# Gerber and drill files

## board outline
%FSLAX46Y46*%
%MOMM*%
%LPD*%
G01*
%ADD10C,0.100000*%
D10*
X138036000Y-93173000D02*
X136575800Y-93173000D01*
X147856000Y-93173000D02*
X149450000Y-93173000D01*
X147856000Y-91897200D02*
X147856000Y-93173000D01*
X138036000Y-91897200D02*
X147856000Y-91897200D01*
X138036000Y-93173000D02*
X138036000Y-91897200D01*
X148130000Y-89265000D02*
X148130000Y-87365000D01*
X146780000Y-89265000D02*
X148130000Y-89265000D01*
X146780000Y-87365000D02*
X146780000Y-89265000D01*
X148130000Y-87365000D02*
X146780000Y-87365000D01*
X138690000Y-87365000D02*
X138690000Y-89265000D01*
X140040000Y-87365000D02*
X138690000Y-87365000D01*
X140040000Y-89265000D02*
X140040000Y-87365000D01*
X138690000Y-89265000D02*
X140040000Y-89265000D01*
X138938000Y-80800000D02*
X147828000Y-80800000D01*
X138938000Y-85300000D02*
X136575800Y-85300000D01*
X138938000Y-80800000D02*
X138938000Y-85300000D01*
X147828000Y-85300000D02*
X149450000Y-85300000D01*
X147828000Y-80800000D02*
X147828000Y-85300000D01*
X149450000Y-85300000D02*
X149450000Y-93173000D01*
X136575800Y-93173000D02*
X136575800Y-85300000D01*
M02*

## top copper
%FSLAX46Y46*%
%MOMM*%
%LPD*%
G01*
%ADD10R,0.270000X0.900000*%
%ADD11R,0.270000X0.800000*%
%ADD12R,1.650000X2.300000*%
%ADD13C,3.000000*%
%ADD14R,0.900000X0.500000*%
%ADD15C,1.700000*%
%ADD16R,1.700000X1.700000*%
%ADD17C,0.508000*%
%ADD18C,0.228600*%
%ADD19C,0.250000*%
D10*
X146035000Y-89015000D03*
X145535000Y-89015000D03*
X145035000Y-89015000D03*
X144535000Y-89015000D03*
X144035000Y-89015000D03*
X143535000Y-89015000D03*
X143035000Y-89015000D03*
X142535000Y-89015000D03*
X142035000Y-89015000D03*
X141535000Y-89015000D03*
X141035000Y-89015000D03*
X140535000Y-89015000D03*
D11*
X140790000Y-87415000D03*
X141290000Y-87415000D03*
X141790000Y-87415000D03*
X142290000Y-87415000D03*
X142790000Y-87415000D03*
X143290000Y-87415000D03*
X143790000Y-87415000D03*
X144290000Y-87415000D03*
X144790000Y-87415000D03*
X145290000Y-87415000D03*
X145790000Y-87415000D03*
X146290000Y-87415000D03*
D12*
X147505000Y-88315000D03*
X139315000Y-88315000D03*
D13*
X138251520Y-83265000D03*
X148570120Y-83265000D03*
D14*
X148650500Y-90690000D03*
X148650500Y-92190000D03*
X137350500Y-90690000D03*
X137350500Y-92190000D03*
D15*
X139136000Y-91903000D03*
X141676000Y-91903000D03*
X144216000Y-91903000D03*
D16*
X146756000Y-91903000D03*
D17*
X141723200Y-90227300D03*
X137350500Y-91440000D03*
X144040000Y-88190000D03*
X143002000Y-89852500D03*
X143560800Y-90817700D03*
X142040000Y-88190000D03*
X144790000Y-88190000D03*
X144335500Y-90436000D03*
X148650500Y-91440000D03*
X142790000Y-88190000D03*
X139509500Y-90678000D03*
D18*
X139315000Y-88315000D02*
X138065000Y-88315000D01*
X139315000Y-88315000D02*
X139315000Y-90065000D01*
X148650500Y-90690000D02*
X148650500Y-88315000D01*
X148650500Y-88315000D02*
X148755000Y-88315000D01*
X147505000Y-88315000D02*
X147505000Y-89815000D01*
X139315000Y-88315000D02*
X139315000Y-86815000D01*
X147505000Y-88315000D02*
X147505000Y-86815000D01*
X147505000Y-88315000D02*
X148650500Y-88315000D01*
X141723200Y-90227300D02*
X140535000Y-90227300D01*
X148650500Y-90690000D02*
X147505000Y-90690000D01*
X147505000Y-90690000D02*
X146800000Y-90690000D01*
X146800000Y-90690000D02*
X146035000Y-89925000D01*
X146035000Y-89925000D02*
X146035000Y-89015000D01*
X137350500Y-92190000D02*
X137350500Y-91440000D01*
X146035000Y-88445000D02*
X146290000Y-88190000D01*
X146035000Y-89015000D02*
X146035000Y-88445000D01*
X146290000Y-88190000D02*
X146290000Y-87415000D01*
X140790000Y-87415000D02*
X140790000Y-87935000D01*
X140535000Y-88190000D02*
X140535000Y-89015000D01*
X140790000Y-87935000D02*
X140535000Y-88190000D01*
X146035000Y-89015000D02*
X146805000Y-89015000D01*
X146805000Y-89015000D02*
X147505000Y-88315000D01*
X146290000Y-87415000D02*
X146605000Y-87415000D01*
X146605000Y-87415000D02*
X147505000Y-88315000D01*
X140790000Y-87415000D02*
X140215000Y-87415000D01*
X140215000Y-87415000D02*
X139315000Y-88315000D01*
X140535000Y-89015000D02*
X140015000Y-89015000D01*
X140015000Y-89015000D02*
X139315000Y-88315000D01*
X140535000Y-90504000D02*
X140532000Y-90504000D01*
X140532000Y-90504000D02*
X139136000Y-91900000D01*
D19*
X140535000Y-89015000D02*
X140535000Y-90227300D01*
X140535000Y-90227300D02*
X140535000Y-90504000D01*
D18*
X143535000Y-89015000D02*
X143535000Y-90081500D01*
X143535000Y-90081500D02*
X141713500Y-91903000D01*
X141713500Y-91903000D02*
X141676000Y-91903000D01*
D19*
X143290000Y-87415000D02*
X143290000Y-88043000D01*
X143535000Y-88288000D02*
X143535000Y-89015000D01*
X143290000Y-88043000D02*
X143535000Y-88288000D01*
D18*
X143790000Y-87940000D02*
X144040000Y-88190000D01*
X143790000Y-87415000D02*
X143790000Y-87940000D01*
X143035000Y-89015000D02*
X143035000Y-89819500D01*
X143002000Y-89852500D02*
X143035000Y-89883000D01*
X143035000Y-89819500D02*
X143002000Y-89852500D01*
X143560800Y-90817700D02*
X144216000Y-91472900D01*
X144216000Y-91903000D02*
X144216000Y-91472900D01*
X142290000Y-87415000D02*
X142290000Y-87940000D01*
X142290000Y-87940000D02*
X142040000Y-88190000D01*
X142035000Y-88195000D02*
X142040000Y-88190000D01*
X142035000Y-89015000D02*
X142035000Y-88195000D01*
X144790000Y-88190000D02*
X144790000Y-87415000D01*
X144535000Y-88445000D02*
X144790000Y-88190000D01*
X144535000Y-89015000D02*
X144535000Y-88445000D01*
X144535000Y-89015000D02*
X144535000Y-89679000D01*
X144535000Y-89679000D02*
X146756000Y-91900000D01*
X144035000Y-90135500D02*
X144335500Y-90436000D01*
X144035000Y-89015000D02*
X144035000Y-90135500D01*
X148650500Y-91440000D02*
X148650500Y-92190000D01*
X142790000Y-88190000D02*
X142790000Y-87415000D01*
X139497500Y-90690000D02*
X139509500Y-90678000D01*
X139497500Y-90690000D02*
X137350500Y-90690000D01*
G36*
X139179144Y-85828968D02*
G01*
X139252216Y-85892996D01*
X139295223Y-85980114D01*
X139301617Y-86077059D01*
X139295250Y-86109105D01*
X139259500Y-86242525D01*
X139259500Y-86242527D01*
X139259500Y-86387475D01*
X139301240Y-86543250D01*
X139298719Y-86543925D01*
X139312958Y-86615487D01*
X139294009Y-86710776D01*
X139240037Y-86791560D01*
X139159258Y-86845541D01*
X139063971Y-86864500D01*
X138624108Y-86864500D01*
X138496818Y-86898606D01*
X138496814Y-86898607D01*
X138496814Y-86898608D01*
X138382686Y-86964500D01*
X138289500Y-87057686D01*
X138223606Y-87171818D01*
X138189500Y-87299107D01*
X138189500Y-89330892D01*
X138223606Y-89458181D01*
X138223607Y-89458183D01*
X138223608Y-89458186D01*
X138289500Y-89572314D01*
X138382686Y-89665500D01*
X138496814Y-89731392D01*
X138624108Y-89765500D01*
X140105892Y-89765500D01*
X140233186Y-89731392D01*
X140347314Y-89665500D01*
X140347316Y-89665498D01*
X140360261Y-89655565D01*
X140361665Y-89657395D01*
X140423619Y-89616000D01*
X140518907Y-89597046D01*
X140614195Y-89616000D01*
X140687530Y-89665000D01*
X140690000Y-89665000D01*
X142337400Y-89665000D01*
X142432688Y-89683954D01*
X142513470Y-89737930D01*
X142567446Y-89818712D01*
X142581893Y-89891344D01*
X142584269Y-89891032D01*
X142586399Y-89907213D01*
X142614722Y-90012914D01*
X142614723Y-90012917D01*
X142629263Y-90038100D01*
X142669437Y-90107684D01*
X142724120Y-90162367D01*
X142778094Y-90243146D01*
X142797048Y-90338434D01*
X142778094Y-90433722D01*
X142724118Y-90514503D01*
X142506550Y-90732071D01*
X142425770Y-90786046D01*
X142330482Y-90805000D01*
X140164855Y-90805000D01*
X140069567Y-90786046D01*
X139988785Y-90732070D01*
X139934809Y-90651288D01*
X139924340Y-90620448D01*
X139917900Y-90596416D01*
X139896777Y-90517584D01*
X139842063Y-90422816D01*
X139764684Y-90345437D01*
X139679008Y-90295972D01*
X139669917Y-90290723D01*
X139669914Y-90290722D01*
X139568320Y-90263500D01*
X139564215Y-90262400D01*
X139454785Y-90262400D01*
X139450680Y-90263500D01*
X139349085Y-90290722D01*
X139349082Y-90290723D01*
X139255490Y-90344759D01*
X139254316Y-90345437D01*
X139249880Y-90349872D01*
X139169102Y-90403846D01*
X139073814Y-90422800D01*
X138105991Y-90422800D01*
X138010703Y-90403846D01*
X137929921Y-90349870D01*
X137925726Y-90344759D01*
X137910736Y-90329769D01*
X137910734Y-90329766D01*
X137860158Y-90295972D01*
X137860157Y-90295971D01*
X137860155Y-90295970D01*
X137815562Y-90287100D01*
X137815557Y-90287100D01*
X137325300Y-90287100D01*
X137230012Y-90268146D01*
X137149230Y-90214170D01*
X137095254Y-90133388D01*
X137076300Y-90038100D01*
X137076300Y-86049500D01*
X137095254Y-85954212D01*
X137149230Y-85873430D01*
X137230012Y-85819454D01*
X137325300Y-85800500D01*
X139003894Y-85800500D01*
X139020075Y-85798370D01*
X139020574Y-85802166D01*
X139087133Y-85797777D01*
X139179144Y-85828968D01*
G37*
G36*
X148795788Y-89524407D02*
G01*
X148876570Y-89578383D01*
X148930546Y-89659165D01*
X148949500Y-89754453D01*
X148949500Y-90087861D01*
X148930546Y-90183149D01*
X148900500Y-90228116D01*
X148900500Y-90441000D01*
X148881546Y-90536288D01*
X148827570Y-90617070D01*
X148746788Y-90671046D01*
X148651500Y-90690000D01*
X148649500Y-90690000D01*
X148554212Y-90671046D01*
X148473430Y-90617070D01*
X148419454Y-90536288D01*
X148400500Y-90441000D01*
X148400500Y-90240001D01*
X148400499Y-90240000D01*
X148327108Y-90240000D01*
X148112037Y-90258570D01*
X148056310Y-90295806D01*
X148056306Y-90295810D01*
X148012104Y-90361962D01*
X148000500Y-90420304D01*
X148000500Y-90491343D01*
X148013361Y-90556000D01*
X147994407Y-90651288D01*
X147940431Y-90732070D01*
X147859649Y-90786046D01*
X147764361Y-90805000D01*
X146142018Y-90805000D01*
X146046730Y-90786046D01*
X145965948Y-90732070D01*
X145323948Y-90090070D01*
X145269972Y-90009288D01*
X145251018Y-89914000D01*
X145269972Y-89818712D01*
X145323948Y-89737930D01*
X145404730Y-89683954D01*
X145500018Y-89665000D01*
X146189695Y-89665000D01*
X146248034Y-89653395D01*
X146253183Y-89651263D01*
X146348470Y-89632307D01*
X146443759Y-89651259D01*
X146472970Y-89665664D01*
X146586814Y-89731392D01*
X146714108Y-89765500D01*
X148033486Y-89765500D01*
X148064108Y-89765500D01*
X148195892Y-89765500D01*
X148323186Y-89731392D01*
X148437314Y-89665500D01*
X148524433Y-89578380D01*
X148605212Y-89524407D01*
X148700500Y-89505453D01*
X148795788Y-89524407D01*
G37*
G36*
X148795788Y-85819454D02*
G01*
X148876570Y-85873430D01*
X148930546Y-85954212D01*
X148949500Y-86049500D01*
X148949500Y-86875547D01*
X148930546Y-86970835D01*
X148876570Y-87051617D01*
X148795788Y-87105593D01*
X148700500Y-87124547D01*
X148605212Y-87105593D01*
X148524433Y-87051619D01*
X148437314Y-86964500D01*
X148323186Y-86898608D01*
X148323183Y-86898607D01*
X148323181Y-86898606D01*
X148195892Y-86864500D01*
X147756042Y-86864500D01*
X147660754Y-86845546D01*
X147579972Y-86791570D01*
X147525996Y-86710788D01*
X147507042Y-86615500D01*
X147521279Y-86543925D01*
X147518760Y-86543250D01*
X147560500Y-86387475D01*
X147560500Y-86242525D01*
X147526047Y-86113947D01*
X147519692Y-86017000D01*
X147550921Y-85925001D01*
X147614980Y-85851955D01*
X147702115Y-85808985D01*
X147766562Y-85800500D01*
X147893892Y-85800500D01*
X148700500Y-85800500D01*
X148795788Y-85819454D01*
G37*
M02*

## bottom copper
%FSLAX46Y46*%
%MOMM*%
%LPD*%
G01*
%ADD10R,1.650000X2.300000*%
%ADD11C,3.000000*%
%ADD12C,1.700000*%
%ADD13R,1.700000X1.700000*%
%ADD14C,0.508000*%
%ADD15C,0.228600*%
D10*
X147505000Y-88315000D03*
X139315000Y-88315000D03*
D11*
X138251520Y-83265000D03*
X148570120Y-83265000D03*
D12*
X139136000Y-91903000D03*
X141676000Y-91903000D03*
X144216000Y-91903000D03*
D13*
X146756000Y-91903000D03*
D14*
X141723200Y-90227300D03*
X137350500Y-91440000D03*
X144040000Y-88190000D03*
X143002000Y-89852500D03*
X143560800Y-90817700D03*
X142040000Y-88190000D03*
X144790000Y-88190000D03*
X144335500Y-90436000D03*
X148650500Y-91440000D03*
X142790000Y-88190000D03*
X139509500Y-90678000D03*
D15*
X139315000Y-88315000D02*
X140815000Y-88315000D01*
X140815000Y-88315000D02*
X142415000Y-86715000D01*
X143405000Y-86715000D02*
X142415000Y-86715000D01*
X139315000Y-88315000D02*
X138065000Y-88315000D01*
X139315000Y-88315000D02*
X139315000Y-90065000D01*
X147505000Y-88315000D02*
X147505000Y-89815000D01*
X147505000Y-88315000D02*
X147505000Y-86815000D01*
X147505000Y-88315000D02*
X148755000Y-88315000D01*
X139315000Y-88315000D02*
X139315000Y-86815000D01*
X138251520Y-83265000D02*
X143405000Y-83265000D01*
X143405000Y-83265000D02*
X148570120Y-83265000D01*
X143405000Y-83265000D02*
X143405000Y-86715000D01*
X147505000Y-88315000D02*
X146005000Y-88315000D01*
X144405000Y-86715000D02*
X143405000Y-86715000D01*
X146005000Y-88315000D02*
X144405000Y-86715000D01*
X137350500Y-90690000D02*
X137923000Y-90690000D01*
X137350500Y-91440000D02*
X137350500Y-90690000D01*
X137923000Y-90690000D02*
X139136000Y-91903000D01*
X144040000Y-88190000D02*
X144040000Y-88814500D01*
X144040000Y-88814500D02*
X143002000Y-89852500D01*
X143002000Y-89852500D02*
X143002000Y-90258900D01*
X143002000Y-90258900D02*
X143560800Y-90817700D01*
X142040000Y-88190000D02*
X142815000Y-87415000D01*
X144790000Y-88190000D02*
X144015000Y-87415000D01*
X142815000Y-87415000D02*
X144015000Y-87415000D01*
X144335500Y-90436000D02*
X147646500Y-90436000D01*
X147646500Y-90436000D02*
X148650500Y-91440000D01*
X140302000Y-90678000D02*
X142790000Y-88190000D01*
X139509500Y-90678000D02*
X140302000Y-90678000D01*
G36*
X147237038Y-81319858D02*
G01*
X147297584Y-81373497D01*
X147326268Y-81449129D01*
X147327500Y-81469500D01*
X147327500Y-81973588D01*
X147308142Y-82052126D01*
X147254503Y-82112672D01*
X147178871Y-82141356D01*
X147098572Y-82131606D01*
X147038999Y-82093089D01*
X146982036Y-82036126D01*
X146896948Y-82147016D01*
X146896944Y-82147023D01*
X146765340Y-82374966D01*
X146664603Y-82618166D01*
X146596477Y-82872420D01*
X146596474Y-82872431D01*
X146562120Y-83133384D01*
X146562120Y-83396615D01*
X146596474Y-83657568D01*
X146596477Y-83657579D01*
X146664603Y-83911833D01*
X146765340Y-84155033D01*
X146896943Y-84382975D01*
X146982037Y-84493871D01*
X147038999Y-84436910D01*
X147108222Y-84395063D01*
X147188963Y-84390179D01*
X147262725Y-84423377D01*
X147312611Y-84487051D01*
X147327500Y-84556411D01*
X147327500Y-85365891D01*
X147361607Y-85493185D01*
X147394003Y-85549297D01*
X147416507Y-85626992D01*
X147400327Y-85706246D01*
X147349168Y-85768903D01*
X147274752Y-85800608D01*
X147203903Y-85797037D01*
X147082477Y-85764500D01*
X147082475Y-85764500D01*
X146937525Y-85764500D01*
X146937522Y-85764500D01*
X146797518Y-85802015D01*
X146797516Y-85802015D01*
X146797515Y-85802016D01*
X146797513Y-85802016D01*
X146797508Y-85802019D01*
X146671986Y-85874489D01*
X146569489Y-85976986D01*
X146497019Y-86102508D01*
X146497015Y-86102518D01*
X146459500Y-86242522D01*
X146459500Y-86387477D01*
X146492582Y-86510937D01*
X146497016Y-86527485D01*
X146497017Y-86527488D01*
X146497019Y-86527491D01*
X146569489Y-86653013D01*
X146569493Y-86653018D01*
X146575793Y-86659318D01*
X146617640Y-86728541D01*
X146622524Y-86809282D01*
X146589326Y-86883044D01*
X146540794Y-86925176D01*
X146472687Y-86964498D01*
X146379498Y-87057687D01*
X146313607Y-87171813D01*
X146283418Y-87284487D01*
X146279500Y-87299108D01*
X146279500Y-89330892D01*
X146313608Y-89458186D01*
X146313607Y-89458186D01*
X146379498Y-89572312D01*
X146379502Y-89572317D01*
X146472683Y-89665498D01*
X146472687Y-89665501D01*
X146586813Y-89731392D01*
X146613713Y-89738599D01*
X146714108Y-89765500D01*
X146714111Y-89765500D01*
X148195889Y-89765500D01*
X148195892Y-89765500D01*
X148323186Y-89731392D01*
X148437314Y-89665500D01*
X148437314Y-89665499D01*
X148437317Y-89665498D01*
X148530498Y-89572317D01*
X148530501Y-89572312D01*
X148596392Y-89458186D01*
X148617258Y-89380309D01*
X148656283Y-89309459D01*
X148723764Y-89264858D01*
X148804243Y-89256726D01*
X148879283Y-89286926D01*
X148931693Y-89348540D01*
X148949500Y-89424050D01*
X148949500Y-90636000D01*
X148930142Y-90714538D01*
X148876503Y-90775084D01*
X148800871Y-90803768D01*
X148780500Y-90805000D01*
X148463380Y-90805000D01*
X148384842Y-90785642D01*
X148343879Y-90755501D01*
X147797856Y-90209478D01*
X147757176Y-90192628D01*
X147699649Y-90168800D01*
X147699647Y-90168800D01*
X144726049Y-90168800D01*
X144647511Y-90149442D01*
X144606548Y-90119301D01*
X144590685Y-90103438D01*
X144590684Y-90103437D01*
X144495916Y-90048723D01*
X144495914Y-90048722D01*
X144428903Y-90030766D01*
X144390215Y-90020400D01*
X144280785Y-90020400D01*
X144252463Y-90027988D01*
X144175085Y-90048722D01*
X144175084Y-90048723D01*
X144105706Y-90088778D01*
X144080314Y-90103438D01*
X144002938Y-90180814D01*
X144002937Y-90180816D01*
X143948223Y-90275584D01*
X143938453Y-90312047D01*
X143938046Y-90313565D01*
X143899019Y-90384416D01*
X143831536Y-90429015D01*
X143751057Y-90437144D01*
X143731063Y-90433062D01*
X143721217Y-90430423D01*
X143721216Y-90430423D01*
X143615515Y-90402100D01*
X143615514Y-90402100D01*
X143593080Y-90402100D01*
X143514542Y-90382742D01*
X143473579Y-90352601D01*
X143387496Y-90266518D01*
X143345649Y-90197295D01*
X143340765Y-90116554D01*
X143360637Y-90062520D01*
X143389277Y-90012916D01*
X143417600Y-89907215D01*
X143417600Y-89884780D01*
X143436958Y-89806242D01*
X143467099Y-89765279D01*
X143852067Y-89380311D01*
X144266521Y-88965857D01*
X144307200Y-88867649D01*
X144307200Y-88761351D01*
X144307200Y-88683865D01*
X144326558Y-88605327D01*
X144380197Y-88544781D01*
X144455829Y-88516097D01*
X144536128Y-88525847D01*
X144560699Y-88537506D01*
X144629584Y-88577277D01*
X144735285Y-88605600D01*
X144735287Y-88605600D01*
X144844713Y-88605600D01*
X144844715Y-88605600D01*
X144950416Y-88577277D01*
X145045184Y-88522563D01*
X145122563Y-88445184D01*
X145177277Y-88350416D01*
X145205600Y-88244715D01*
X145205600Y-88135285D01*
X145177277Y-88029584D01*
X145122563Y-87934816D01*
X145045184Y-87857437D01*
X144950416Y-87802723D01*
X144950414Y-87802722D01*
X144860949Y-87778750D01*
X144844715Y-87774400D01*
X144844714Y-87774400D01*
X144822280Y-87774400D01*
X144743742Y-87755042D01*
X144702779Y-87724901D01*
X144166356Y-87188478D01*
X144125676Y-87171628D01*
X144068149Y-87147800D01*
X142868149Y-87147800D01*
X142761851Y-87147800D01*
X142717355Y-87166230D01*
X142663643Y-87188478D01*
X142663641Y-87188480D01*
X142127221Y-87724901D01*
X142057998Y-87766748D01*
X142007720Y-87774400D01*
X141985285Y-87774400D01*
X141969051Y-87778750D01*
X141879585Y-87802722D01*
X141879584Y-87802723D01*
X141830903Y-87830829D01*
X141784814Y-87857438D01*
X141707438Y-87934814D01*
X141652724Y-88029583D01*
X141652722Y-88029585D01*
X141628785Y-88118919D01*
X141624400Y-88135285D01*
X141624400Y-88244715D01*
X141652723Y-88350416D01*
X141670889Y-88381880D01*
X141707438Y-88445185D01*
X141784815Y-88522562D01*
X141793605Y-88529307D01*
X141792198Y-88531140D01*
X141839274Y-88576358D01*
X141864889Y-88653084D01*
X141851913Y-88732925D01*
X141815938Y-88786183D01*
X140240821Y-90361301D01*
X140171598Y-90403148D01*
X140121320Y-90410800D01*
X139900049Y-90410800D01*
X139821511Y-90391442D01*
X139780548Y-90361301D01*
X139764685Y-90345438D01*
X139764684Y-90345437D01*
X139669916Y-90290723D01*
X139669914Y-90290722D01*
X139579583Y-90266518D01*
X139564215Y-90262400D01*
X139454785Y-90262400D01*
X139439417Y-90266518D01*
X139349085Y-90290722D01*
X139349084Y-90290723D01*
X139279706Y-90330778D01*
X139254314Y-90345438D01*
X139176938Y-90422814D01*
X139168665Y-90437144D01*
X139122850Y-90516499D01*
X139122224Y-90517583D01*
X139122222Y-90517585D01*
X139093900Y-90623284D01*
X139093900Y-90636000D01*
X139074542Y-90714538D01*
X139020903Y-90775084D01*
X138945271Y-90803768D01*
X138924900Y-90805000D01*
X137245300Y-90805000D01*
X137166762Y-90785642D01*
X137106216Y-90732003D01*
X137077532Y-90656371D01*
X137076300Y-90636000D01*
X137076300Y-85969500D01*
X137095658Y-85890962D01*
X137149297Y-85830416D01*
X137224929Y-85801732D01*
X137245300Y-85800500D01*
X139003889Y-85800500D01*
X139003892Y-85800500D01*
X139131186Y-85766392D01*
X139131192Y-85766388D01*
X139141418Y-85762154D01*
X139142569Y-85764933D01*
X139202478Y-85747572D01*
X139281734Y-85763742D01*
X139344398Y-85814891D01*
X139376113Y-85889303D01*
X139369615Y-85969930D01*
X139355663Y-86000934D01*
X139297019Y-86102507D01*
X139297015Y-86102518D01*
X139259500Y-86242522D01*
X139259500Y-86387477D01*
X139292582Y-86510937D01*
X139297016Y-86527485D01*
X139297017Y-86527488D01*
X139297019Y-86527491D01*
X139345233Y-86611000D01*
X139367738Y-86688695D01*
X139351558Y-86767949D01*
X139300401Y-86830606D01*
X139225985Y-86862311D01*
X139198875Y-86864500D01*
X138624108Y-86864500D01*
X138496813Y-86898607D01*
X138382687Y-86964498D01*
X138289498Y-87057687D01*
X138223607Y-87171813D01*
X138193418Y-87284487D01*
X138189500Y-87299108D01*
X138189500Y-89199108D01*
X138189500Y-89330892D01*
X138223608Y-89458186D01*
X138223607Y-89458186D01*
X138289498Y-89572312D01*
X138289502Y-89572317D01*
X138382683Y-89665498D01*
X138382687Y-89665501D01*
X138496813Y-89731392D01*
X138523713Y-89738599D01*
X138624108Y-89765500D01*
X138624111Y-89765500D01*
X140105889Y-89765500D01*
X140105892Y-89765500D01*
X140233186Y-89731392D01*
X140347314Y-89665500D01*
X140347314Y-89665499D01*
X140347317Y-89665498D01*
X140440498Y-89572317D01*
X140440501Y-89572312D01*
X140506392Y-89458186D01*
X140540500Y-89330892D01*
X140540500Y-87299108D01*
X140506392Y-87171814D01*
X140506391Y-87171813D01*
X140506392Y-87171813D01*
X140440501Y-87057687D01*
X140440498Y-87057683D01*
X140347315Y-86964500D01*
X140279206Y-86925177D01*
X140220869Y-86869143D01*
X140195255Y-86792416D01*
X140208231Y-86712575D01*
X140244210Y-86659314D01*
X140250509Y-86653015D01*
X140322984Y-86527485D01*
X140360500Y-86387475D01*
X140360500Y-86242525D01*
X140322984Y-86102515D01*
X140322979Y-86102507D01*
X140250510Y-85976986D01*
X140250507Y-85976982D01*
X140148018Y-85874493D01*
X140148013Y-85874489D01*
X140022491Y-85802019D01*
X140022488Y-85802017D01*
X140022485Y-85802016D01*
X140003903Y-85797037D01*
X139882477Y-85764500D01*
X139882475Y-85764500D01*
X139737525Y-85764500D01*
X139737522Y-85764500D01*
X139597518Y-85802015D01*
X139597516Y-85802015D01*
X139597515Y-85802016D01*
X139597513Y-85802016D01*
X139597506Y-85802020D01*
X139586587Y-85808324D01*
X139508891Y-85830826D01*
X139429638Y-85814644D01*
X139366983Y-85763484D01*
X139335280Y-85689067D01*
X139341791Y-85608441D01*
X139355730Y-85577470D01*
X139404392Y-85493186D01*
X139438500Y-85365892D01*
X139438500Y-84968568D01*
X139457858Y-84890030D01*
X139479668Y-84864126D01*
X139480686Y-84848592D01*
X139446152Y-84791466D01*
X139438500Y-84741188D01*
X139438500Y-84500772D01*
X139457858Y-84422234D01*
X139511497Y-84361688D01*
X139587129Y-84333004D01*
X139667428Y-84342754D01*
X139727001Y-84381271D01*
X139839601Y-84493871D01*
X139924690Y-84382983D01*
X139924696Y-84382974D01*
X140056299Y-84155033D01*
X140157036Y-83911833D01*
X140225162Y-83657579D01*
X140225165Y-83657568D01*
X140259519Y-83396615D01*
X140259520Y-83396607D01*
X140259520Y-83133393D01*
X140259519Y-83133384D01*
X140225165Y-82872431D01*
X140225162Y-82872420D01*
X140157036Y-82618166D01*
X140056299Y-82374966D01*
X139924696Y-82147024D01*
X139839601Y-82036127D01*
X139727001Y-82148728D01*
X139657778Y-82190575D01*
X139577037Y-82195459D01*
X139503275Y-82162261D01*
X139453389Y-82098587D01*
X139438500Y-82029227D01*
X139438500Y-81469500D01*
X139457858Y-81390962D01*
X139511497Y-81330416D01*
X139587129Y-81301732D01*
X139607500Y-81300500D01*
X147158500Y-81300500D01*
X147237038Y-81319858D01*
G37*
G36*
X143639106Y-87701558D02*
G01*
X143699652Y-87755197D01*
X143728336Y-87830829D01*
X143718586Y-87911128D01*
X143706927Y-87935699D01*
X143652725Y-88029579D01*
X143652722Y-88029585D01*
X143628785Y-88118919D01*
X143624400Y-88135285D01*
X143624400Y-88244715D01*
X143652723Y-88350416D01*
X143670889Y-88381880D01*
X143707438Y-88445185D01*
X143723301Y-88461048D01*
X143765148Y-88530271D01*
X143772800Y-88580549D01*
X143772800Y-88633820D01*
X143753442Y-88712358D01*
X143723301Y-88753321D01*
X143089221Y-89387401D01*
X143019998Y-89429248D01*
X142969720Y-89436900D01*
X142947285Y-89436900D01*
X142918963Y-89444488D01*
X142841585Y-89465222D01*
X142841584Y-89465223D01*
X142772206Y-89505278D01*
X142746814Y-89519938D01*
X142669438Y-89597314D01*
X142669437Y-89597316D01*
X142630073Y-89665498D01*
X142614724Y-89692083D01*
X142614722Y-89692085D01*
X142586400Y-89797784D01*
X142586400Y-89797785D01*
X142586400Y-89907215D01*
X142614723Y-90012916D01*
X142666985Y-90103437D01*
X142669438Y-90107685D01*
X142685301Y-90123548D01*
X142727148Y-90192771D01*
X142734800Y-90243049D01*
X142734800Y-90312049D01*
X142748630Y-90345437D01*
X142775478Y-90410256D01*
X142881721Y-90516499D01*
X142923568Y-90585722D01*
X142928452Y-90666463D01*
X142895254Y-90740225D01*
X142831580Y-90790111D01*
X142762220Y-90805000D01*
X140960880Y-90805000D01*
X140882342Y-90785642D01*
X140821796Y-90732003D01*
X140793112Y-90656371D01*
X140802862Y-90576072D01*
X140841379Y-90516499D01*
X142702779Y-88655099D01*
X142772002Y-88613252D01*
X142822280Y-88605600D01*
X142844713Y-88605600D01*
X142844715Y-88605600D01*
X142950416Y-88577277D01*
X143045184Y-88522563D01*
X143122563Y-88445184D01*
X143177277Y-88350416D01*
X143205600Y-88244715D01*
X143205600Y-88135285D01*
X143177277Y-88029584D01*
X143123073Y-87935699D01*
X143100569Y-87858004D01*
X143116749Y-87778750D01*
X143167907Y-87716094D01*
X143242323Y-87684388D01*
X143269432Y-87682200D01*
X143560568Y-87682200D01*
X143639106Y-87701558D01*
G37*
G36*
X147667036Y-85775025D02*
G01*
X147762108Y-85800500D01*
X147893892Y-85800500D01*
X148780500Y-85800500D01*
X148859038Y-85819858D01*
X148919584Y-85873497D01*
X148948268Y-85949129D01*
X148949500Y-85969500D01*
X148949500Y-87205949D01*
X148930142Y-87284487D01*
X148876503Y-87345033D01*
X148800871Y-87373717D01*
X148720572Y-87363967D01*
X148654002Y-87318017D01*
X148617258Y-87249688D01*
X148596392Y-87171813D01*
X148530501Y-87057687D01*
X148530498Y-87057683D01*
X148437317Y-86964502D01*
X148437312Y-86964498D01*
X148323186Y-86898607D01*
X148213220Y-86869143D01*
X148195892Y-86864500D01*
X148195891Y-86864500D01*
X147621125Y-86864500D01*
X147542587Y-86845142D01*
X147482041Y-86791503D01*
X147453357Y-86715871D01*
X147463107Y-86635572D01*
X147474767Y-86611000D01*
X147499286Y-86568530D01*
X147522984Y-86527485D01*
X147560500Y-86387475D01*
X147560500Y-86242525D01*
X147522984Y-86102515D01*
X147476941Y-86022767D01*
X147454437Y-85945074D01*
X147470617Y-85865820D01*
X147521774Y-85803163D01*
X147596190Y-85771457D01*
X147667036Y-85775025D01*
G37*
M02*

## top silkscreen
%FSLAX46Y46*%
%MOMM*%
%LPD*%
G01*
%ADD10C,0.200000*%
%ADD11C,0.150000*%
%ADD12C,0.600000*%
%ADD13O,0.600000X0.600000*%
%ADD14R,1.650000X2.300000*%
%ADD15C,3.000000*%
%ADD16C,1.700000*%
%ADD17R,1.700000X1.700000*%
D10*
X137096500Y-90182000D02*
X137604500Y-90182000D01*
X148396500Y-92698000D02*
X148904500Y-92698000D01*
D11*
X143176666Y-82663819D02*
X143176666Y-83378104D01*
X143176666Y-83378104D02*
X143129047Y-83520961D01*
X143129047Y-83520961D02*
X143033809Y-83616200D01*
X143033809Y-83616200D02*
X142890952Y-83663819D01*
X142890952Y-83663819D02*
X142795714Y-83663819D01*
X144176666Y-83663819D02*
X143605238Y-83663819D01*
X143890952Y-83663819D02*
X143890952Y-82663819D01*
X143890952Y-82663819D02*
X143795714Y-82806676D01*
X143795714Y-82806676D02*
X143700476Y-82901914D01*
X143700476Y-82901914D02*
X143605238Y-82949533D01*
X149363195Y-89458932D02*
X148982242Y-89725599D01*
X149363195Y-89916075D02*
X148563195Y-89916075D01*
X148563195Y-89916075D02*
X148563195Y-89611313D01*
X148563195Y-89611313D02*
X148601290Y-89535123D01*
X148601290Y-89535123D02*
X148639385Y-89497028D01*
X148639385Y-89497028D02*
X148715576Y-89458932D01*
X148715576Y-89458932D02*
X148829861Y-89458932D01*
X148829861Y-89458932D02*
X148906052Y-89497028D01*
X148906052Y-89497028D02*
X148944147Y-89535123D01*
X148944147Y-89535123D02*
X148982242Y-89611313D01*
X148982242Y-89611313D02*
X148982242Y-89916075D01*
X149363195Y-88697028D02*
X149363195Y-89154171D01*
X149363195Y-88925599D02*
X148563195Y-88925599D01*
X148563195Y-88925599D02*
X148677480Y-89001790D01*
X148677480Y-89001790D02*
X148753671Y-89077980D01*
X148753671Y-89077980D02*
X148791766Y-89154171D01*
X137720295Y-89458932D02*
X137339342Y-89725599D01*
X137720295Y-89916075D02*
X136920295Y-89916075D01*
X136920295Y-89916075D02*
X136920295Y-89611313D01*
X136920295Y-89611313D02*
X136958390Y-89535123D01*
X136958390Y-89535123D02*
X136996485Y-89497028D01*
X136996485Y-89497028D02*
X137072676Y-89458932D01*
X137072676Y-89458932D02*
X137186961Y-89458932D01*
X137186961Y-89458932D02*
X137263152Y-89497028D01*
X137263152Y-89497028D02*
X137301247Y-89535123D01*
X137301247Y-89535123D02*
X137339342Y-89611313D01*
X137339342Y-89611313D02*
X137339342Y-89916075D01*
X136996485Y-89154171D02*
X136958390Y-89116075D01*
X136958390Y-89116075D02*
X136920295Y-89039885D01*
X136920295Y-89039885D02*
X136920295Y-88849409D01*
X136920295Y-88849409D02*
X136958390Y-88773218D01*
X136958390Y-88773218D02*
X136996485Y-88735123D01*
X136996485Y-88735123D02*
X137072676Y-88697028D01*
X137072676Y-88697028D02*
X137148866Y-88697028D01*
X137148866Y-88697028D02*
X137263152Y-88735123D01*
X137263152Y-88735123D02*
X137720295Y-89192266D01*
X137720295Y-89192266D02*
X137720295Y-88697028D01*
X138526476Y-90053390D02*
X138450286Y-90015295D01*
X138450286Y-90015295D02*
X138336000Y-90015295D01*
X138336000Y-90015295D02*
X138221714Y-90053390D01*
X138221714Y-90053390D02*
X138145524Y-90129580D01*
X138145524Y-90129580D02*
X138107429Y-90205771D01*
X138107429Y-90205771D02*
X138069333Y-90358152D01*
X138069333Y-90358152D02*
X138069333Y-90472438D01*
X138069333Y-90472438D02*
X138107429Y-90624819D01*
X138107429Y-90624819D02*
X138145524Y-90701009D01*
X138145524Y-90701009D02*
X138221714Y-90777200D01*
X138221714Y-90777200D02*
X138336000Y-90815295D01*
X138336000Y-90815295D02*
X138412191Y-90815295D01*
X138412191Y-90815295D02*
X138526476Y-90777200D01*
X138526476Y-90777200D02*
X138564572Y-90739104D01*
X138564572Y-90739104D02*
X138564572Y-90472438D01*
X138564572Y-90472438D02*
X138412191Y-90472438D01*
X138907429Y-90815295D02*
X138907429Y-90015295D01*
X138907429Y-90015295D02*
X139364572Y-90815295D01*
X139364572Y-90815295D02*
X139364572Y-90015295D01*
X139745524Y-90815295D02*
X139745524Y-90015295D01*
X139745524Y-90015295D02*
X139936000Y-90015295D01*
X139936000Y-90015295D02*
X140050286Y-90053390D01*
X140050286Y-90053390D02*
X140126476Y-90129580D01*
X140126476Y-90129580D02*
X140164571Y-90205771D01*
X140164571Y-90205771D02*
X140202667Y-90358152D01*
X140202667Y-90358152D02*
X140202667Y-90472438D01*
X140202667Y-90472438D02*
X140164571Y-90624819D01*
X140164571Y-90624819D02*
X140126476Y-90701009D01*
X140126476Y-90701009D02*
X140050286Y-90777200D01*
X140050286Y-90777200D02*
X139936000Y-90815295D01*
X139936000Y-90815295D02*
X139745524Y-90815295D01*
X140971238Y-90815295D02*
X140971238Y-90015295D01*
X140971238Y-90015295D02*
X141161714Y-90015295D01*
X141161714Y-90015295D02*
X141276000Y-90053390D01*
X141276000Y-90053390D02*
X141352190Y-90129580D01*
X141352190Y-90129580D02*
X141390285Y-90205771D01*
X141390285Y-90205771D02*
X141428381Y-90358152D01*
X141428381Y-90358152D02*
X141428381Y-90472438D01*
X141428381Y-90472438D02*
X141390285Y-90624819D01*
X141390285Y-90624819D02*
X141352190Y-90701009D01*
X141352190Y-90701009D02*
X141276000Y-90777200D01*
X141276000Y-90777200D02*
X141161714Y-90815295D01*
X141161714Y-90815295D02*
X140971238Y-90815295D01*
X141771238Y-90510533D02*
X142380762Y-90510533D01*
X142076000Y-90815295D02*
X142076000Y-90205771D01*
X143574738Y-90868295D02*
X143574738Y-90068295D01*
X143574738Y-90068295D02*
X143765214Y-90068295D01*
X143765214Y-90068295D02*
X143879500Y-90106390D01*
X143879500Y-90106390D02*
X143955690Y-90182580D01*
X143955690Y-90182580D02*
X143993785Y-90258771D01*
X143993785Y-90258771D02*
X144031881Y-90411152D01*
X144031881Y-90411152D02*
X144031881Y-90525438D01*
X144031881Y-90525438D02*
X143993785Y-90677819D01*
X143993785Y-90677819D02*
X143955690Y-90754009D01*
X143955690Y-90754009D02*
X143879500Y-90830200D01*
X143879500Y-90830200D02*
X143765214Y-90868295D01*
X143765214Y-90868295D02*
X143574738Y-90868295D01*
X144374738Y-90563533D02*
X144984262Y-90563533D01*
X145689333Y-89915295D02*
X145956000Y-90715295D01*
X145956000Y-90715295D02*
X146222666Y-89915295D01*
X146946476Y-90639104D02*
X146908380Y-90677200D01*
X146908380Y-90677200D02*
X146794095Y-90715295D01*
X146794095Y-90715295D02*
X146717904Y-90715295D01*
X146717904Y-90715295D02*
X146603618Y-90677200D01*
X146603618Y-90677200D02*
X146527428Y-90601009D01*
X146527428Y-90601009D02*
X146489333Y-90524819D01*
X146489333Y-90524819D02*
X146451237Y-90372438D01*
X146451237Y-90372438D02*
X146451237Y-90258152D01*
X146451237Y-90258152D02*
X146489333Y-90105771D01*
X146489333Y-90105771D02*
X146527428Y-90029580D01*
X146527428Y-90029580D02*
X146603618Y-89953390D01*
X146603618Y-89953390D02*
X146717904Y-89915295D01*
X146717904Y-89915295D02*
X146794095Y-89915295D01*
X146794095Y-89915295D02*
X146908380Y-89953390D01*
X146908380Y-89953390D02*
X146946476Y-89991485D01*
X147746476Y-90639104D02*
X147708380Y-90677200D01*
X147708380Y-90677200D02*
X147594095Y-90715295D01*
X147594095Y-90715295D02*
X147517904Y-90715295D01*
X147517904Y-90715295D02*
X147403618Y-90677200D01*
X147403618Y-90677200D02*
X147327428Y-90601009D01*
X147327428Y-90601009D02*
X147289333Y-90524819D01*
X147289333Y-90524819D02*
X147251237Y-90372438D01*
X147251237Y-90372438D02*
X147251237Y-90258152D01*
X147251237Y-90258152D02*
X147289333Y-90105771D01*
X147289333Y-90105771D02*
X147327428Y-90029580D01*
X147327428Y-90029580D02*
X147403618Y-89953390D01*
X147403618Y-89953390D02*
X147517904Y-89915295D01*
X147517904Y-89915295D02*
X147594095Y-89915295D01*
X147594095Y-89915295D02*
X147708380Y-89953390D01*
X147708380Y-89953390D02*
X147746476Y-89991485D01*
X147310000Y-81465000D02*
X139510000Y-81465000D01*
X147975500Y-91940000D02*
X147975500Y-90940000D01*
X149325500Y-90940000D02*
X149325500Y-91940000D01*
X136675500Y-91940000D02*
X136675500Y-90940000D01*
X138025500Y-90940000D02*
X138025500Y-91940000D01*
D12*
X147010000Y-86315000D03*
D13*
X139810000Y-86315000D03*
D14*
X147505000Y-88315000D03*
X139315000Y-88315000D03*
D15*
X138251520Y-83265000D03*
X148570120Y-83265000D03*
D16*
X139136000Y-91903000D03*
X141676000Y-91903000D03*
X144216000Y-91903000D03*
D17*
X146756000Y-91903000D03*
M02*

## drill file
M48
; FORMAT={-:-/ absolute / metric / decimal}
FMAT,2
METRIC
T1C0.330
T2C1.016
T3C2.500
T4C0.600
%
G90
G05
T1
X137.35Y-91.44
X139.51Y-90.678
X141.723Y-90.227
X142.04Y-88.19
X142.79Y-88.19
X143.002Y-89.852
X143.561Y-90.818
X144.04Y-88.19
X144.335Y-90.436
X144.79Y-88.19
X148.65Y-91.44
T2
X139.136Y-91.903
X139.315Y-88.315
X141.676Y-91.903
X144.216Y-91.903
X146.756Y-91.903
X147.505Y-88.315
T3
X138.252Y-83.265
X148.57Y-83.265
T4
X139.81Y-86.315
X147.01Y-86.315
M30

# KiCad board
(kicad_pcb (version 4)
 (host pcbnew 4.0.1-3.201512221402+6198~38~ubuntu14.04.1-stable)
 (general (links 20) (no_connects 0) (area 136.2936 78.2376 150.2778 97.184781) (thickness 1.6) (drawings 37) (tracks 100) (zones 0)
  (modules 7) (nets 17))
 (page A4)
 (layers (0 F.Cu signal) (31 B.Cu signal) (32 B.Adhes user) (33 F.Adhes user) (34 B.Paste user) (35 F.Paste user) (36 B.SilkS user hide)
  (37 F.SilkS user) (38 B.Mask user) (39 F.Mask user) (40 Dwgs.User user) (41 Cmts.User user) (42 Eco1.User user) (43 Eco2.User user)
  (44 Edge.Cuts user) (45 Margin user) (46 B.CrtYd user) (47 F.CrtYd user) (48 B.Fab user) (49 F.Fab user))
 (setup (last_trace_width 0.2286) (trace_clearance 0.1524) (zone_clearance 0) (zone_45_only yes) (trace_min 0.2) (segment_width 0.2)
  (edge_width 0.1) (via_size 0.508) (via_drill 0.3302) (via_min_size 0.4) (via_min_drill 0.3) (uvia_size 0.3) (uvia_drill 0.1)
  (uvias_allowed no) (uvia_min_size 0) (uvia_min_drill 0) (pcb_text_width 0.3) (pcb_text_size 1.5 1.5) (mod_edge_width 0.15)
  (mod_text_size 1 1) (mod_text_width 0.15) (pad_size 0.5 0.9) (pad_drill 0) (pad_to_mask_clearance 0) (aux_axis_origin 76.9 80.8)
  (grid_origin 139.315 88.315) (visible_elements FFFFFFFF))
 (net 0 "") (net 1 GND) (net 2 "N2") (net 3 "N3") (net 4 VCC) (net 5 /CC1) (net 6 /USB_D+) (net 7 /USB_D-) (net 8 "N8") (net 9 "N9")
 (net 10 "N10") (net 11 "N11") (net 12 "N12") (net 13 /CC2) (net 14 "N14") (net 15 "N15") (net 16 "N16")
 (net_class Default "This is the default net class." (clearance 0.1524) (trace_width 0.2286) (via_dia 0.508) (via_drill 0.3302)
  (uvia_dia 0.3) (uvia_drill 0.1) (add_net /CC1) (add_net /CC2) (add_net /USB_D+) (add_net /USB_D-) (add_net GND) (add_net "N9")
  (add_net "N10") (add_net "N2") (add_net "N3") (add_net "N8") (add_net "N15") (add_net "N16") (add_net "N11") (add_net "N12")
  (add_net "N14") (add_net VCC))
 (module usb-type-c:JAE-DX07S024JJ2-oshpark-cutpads (layer F.Cu) (at 147.01 86.315 180)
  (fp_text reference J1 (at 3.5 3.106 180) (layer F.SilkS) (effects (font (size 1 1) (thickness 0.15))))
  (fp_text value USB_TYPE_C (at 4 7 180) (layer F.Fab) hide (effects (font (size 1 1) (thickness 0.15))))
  (fp_line (start -0.3 4.85) (end 7.5 4.85) (layer F.SilkS) (width 0.15))
  (pad A1 smd rect (at 0.975 -2.7 180) (size 0.27 0.9) (layers F.Cu F.Paste F.Mask) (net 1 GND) (zone_connect 1) (thermal_width 0.2)
   (thermal_gap 0.2))
  (pad A2 smd rect (at 1.475 -2.7 180) (size 0.27 0.9) (layers F.Cu F.Paste F.Mask) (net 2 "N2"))
  (pad A3 smd rect (at 1.975 -2.7 180) (size 0.27 0.9) (layers F.Cu F.Paste F.Mask) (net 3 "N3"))
  (pad A4 smd rect (at 2.475 -2.7 180) (size 0.27 0.9) (layers F.Cu F.Paste F.Mask) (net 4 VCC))
  (pad A5 smd rect (at 2.975 -2.7 180) (size 0.27 0.9) (layers F.Cu F.Paste F.Mask) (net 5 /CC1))
  (pad A6 smd rect (at 3.475 -2.7 180) (size 0.27 0.9) (layers F.Cu F.Paste F.Mask) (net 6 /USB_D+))
  (pad A7 smd rect (at 3.975 -2.7 180) (size 0.27 0.9) (layers F.Cu F.Paste F.Mask) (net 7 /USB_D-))
  (pad A8 smd rect (at 4.475 -2.7 180) (size 0.27 0.9) (layers F.Cu F.Paste F.Mask) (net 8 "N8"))
  (pad A9 smd rect (at 4.975 -2.7 180) (size 0.27 0.9) (layers F.Cu F.Paste F.Mask) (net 4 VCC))
  (pad A10 smd rect (at 5.475 -2.7 180) (size 0.27 0.9) (layers F.Cu F.Paste F.Mask) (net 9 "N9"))
  (pad A11 smd rect (at 5.975 -2.7 180) (size 0.27 0.9) (layers F.Cu F.Paste F.Mask) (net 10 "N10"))
  (pad A12 smd rect (at 6.475 -2.7 180) (size 0.27 0.9) (layers F.Cu F.Paste F.Mask) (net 1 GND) (zone_connect 2))
  (pad B1 smd rect (at 6.22 -1.1 180) (size 0.27 0.8) (layers F.Cu F.Paste F.Mask) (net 1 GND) (zone_connect 2))
  (pad B2 smd rect (at 5.72 -1.1 180) (size 0.27 0.8) (layers F.Cu F.Paste F.Mask) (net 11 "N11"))
  (pad B3 smd rect (at 5.22 -1.1 180) (size 0.27 0.8) (layers F.Cu F.Paste F.Mask) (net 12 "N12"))
  (pad B4 smd rect (at 4.72 -1.1 180) (size 0.27 0.8) (layers F.Cu F.Paste F.Mask) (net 4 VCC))
  (pad B5 smd rect (at 4.22 -1.1 180) (size 0.27 0.8) (layers F.Cu F.Paste F.Mask) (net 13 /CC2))
  (pad B6 smd rect (at 3.72 -1.1 180) (size 0.27 0.8) (layers F.Cu F.Paste F.Mask) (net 6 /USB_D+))
  (pad B7 smd rect (at 3.22 -1.1 180) (size 0.27 0.8) (layers F.Cu F.Paste F.Mask) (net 7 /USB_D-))
  (pad B8 smd rect (at 2.72 -1.1 180) (size 0.27 0.8) (layers F.Cu F.Paste F.Mask) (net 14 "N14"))
  (pad B9 smd rect (at 2.22 -1.1 180) (size 0.27 0.8) (layers F.Cu F.Paste F.Mask) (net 4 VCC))
  (pad B10 smd rect (at 1.72 -1.1 180) (size 0.27 0.8) (layers F.Cu F.Paste F.Mask) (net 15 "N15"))
  (pad B11 smd rect (at 1.22 -1.1 180) (size 0.27 0.8) (layers F.Cu F.Paste F.Mask) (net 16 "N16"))
  (pad B12 smd rect (at 0.72 -1.1 180) (size 0.27 0.8) (layers F.Cu F.Paste F.Mask) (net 1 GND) (zone_connect 2))
  (pad "" np_thru_hole circle (at 0 0 180) (size 0.6 0.6) (drill 0.6) (layers *.Cu *.Mask F.SilkS))
  (pad "" np_thru_hole oval (at 7.2 0 180) (size 0.6 0.6) (drill 0.6) (layers *.Cu *.Mask F.SilkS))
  (pad 0 thru_hole rect (at -0.495 -2 180) (size 1.65 2.3) (drill 1.016) (layers *.Cu *.Mask F.SilkS) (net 1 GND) (zone_connect 1)
   (thermal_width 0.2) (thermal_gap 0.2))
  (pad 0 thru_hole rect (at 7.695 -2 180) (size 1.65 2.3) (drill 1.016) (layers *.Cu *.Mask F.SilkS) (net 1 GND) (zone_connect 1)
   (thermal_width 0.2) (thermal_gap 0.2))
  (pad 0 thru_hole circle (at 8.75848 3.05 180) (size 3 3) (drill 2.5) (layers *.Cu *.Mask F.SilkS) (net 1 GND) (zone_connect 1))
  (pad 0 thru_hole circle (at -1.56012 3.05 180) (size 3 3) (drill 2.5) (layers *.Cu *.Mask F.SilkS) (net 1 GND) (zone_connect 1)))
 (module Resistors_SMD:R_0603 (layer F.Cu) (at 148.6505 91.44 270)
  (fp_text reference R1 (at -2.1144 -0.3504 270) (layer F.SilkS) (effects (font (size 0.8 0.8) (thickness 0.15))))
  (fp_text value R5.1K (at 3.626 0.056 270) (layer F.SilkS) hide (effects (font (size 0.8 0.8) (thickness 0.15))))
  (fp_line (start 0.5 0.675) (end -0.5 0.675) (layer F.SilkS) (width 0.15))
  (fp_line (start -0.5 -0.675) (end 0.5 -0.675) (layer F.SilkS) (width 0.15))
  (pad 1 smd rect (at -0.75 0 270) (size 0.5 0.9) (layers F.Cu F.Paste F.Mask) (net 1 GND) (zone_connect 1) (thermal_width 0.2)
   (thermal_gap 0.2))
  (pad 2 smd rect (at 0.75 0 270) (size 0.5 0.9) (layers F.Cu F.Paste F.Mask) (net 5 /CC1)))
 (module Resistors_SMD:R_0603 (layer F.Cu) (at 137.3505 91.44 270)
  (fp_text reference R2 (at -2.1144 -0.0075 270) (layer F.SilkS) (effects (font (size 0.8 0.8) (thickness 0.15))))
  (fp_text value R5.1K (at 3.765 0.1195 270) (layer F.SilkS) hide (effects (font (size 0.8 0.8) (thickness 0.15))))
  (fp_line (start 0.5 0.675) (end -0.5 0.675) (layer F.SilkS) (width 0.15))
  (fp_line (start -0.5 -0.675) (end 0.5 -0.675) (layer F.SilkS) (width 0.15))
  (pad 1 smd rect (at -0.75 0 270) (size 0.5 0.9) (layers F.Cu F.Paste F.Mask) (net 13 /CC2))
  (pad 2 smd rect (at 0.75 0 270) (size 0.5 0.9) (layers F.Cu F.Paste F.Mask) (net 1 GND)))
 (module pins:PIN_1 (layer F.Cu) (at 139.136 91.903)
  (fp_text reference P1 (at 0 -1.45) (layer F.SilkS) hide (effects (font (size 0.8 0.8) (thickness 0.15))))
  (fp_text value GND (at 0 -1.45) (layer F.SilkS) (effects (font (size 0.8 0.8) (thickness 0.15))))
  (pad 1 thru_hole circle (at 0 0) (size 1.7 1.7) (drill 1.016) (layers *.Cu *.Mask F.SilkS) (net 1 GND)))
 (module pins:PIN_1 (layer F.Cu) (at 141.676 91.903)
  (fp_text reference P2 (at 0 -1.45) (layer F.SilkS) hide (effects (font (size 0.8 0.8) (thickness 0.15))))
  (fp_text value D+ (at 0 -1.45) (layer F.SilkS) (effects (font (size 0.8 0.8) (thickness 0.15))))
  (pad 1 thru_hole circle (at 0 0) (size 1.7 1.7) (drill 1.016) (layers *.Cu *.Mask F.SilkS) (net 6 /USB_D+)))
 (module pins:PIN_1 (layer F.Cu) (at 144.216 91.903 90)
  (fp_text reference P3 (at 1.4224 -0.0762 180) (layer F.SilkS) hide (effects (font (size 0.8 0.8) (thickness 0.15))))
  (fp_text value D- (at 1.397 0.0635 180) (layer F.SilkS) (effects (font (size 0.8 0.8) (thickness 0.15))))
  (pad 1 thru_hole circle (at 0 0 90) (size 1.7 1.7) (drill 1.016) (layers *.Cu *.Mask F.SilkS) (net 7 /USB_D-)))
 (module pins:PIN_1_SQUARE (layer F.Cu) (at 146.756 91.903)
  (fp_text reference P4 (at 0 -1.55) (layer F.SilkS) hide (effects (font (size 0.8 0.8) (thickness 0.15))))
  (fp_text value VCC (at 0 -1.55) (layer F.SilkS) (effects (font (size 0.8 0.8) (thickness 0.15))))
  (pad 1 thru_hole rect (at 0 0) (size 1.7 1.7) (drill 1.016) (layers *.Cu *.Mask F.SilkS) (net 4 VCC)))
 (gr_line (start 137.0965 90.182) (end 137.6045 90.182) (angle 90) (layer F.SilkS) (width 0.2))
 (gr_line (start 148.3965 92.698) (end 148.9045 92.698) (angle 90) (layer F.SilkS) (width 0.2))
 (gr_line (start 138.036 93.173) (end 136.5758 93.173) (angle 90) (layer Edge.Cuts) (width 0.1))
 (gr_line (start 147.856 93.173) (end 149.45 93.173) (angle 90) (layer Edge.Cuts) (width 0.1))
 (gr_line (start 147.856 91.8972) (end 147.856 93.173) (angle 90) (layer Edge.Cuts) (width 0.1))
 (gr_line (start 138.036 91.8972) (end 147.856 91.8972) (angle 90) (layer Edge.Cuts) (width 0.1))
 (gr_line (start 138.036 93.173) (end 138.036 91.8972) (angle 90) (layer Edge.Cuts) (width 0.1))
 (gr_line (start 148.13 89.265) (end 148.13 87.365) (angle 90) (layer Edge.Cuts) (width 0.1))
 (gr_line (start 146.78 89.265) (end 148.13 89.265) (angle 90) (layer Edge.Cuts) (width 0.1))
 (gr_line (start 146.78 87.365) (end 146.78 89.265) (angle 90) (layer Edge.Cuts) (width 0.1))
 (gr_line (start 148.13 87.365) (end 146.78 87.365) (angle 90) (layer Edge.Cuts) (width 0.1))
 (gr_line (start 138.69 87.365) (end 138.69 89.265) (angle 90) (layer Edge.Cuts) (width 0.1))
 (gr_line (start 140.04 87.365) (end 138.69 87.365) (angle 90) (layer Edge.Cuts) (width 0.1))
 (gr_line (start 140.04 89.265) (end 140.04 87.365) (angle 90) (layer Edge.Cuts) (width 0.1))
 (gr_line (start 138.69 89.265) (end 140.04 89.265) (angle 90) (layer Edge.Cuts) (width 0.1))
 (gr_line (start 138.938 80.8) (end 147.828 80.8) (angle 90) (layer Edge.Cuts) (width 0.1))
 (gr_line (start 138.938 85.3) (end 136.5758 85.3) (angle 90) (layer Edge.Cuts) (width 0.1))
 (gr_line (start 138.938 80.8) (end 138.938 85.3) (angle 90) (layer Edge.Cuts) (width 0.1))
 (gr_line (start 147.828 85.3) (end 149.45 85.3) (angle 90) (layer Edge.Cuts) (width 0.1))
 (gr_line (start 147.828 80.8) (end 147.828 85.3) (angle 90) (layer Edge.Cuts) (width 0.1))
 (gr_line (start 149.45 85.3) (end 149.45 93.173) (angle 90) (layer Edge.Cuts) (width 0.1))
 (gr_line (start 136.5758 93.173) (end 136.5758 85.3) (angle 90) (layer Edge.Cuts) (width 0.1))
 (segment (start 139.315 88.315) (end 140.815 88.315) (width 0.2286) (layer B.Cu) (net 1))
 (segment (start 140.815 88.315) (end 142.415 86.715) (width 0.2286) (layer B.Cu) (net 1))
 (segment (start 143.405 86.715) (end 142.415 86.715) (width 0.2286) (layer B.Cu) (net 1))
 (segment (start 139.315 88.315) (end 138.065 88.315) (width 0.2286) (layer B.Cu) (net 1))
 (segment (start 139.315 88.315) (end 138.065 88.315) (width 0.2286) (layer F.Cu) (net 1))
 (segment (start 139.315 88.315) (end 139.315 90.065) (width 0.2286) (layer B.Cu) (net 1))
 (segment (start 147.505 88.315) (end 147.505 89.815) (width 0.2286) (layer B.Cu) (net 1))
 (segment (start 147.505 88.315) (end 147.505 86.815) (width 0.2286) (layer B.Cu) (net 1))
 (segment (start 147.505 88.315) (end 148.755 88.315) (width 0.2286) (layer B.Cu) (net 1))
 (segment (start 139.315 88.315) (end 139.315 86.815) (width 0.2286) (layer B.Cu) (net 1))
 (segment (start 138.25152 83.265) (end 143.405 83.265) (width 0.2286) (layer B.Cu) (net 1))
 (segment (start 143.405 83.265) (end 148.57012 83.265) (width 0.2286) (layer B.Cu) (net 1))
 (segment (start 143.405 83.265) (end 143.405 86.715) (width 0.2286) (layer B.Cu) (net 1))
 (segment (start 147.505 88.315) (end 146.005 88.315) (width 0.2286) (layer B.Cu) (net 1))
 (segment (start 144.405 86.715) (end 143.405 86.715) (width 0.2286) (layer B.Cu) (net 1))
 (segment (start 146.005 88.315) (end 144.405 86.715) (width 0.2286) (layer B.Cu) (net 1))
 (segment (start 139.315 88.315) (end 139.315 90.065) (width 0.2286) (layer F.Cu) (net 1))
 (segment (start 148.6505 90.69) (end 148.6505 88.315) (width 0.2286) (layer F.Cu) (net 1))
 (segment (start 148.6505 88.315) (end 148.755 88.315) (width 0.2286) (layer F.Cu) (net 1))
 (segment (start 147.505 88.315) (end 147.505 89.815) (width 0.2286) (layer F.Cu) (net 1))
 (segment (start 139.315 88.315) (end 139.315 86.815) (width 0.2286) (layer F.Cu) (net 1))
 (segment (start 147.505 88.315) (end 147.505 86.815) (width 0.2286) (layer F.Cu) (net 1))
 (segment (start 147.505 88.315) (end 148.6505 88.315) (width 0.2286) (layer F.Cu) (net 1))
 (via (at 141.7232 90.2273) (size 0.508) (drill 0.3302) (layers F.Cu B.Cu) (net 1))
 (segment (start 141.7232 90.2273) (end 140.535 90.2273) (width 0.2286) (layer F.Cu) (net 1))
 (segment (start 148.6505 90.69) (end 147.505 90.69) (width 0.2286) (layer F.Cu) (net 1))
 (segment (start 147.505 90.69) (end 146.8 90.69) (width 0.2286) (layer F.Cu) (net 1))
 (segment (start 146.8 90.69) (end 146.035 89.925) (width 0.2286) (layer F.Cu) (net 1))
 (segment (start 146.035 89.925) (end 146.035 89.015) (width 0.2286) (layer F.Cu) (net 1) (status 20))
 (segment (start 137.3505 90.69) (end 137.923 90.69) (width 0.2286) (layer B.Cu) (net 1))
 (via (at 137.3505 91.44) (size 0.508) (drill 0.3302) (layers F.Cu B.Cu) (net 1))
 (segment (start 137.3505 91.44) (end 137.3505 90.69) (width 0.2286) (layer B.Cu) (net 1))
 (segment (start 137.3505 92.19) (end 137.3505 91.44) (width 0.2286) (layer F.Cu) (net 1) (status 10))
 (segment (start 137.923 90.69) (end 139.136 91.903) (width 0.2286) (layer B.Cu) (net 1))
 (segment (start 146.035 88.445) (end 146.29 88.19) (width 0.2286) (layer F.Cu) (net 1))
 (segment (start 146.035 89.015) (end 146.035 88.445) (width 0.2286) (layer F.Cu) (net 1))
 (segment (start 146.29 88.19) (end 146.29 87.415) (width 0.2286) (layer F.Cu) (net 1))
 (segment (start 140.79 87.415) (end 140.79 87.935) (width 0.2286) (layer F.Cu) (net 1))
 (segment (start 140.535 88.19) (end 140.535 89.015) (width 0.2286) (layer F.Cu) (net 1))
 (segment (start 140.79 87.935) (end 140.535 88.19) (width 0.2286) (layer F.Cu) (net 1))
 (segment (start 146.035 89.015) (end 146.805 89.015) (width 0.2286) (layer F.Cu) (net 1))
 (segment (start 146.805 89.015) (end 147.505 88.315) (width 0.2286) (layer F.Cu) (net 1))
 (segment (start 146.29 87.415) (end 146.605 87.415) (width 0.2286) (layer F.Cu) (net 1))
 (segment (start 146.605 87.415) (end 147.505 88.315) (width 0.2286) (layer F.Cu) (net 1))
 (segment (start 140.79 87.415) (end 140.215 87.415) (width 0.2286) (layer F.Cu) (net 1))
 (segment (start 140.215 87.415) (end 139.315 88.315) (width 0.2286) (layer F.Cu) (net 1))
 (segment (start 140.535 89.015) (end 140.015 89.015) (width 0.2286) (layer F.Cu) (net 1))
 (segment (start 140.015 89.015) (end 139.315 88.315) (width 0.2286) (layer F.Cu) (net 1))
 (segment (start 140.535 90.504) (end 140.532 90.504) (width 0.2286) (layer F.Cu) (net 1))
 (segment (start 140.532 90.504) (end 139.136 91.9) (width 0.2286) (layer F.Cu) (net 1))
 (segment (start 140.535 89.015) (end 140.535 90.2273) (width 0.25) (layer F.Cu) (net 1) (status 10))
 (segment (start 140.535 90.2273) (end 140.535 90.504) (width 0.25) (layer F.Cu) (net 1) (status 10))
 (segment (start 143.535 89.015) (end 143.535 90.0815) (width 0.2286) (layer F.Cu) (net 6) (status 10))
 (segment (start 143.535 90.0815) (end 141.7135 91.903) (width 0.2286) (layer F.Cu) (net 6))
 (segment (start 141.7135 91.903) (end 141.676 91.903) (width 0.2286) (layer F.Cu) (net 6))
 (segment (start 143.29 87.415) (end 143.29 88.043) (width 0.25) (layer F.Cu) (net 6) (status 10))
 (segment (start 143.535 88.288) (end 143.535 89.015) (width 0.25) (layer F.Cu) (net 6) (status 20))
 (segment (start 143.29 88.043) (end 143.535 88.288) (width 0.25) (layer F.Cu) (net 6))
 (segment (start 144.04 88.19) (end 144.04 88.8145) (width 0.2286) (layer B.Cu) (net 7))
 (via (at 144.04 88.19) (size 0.508) (drill 0.3302) (layers F.Cu B.Cu) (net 7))
 (segment (start 143.79 87.94) (end 144.04 88.19) (width 0.2286) (layer F.Cu) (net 7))
 (segment (start 143.79 87.415) (end 143.79 87.94) (width 0.2286) (layer F.Cu) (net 7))
 (segment (start 144.04 88.8145) (end 143.002 89.8525) (width 0.2286) (layer B.Cu) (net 7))
 (segment (start 143.035 89.015) (end 143.035 89.8195) (width 0.2286) (layer F.Cu) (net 7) (status 10))
 (segment (start 143.002 89.8525) (end 143.002 90.2589) (width 0.2286) (layer B.Cu) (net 7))
 (segment (start 143.002 89.8525) (end 143.035 89.883) (width 0.2286) (layer F.Cu) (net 7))
 (via (at 143.002 89.8525) (size 0.508) (drill 0.3302) (layers F.Cu B.Cu) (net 7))
 (segment (start 143.035 89.8195) (end 143.002 89.8525) (width 0.2286) (layer F.Cu) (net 7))
 (segment (start 143.002 90.2589) (end 143.5608 90.8177) (width 0.2286) (layer B.Cu) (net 7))
 (segment (start 143.5608 90.8177) (end 144.216 91.4729) (width 0.2286) (layer F.Cu) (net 7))
 (via (at 143.5608 90.8177) (size 0.508) (drill 0.3302) (layers F.Cu B.Cu) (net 7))
 (segment (start 144.216 91.903) (end 144.216 91.4729) (width 0.2286) (layer F.Cu) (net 7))
 (segment (start 142.04 88.19) (end 142.815 87.415) (width 0.2286) (layer B.Cu) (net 4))
 (segment (start 142.29 87.415) (end 142.29 87.94) (width 0.2286) (layer F.Cu) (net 4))
 (segment (start 142.29 87.94) (end 142.04 88.19) (width 0.2286) (layer F.Cu) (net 4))
 (via (at 142.04 88.19) (size 0.508) (drill 0.3302) (layers F.Cu B.Cu) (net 4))
 (segment (start 142.035 88.195) (end 142.04 88.19) (width 0.2286) (layer F.Cu) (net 4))
 (segment (start 142.035 89.015) (end 142.035 88.195) (width 0.2286) (layer F.Cu) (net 4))
 (segment (start 144.79 88.19) (end 144.79 87.415) (width 0.2286) (layer F.Cu) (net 4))
 (via (at 144.79 88.19) (size 0.508) (drill 0.3302) (layers F.Cu B.Cu) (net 4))
 (segment (start 144.79 88.19) (end 144.015 87.415) (width 0.2286) (layer B.Cu) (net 4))
 (segment (start 142.815 87.415) (end 144.015 87.415) (width 0.2286) (layer B.Cu) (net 4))
 (segment (start 144.535 88.445) (end 144.79 88.19) (width 0.2286) (layer F.Cu) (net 4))
 (segment (start 144.535 89.015) (end 144.535 88.445) (width 0.2286) (layer F.Cu) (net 4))
 (segment (start 144.535 89.015) (end 144.535 89.679) (width 0.2286) (layer F.Cu) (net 4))
 (segment (start 144.535 89.679) (end 146.756 91.9) (width 0.2286) (layer F.Cu) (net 4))
 (segment (start 144.3355 90.436) (end 147.6465 90.436) (width 0.2286) (layer B.Cu) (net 5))
 (segment (start 144.035 90.1355) (end 144.3355 90.436) (width 0.2286) (layer F.Cu) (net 5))
 (via (at 144.3355 90.436) (size 0.508) (drill 0.3302) (layers F.Cu B.Cu) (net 5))
 (segment (start 144.035 89.015) (end 144.035 90.1355) (width 0.2286) (layer F.Cu) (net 5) (status 10))
 (via (at 148.6505 91.44) (size 0.508) (drill 0.3302) (layers F.Cu B.Cu) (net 5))
 (segment (start 148.6505 91.44) (end 148.6505 92.19) (width 0.2286) (layer F.Cu) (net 5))
 (segment (start 147.6465 90.436) (end 148.6505 91.44) (width 0.2286) (layer B.Cu) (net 5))
 (segment (start 140.302 90.678) (end 142.79 88.19) (width 0.2286) (layer B.Cu) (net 13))
 (segment (start 139.5095 90.678) (end 140.302 90.678) (width 0.2286) (layer B.Cu) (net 13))
 (via (at 142.79 88.19) (size 0.508) (drill 0.3302) (layers F.Cu B.Cu) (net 13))
 (segment (start 142.79 88.19) (end 142.79 87.415) (width 0.2286) (layer F.Cu) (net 13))
 (via (at 139.5095 90.678) (size 0.508) (drill 0.3302) (layers F.Cu B.Cu) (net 13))
 (segment (start 139.4975 90.69) (end 139.5095 90.678) (width 0.2286) (layer F.Cu) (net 13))
 (segment (start 139.4975 90.69) (end 137.3505 90.69) (width 0.2286) (layer F.Cu) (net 13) (status 20))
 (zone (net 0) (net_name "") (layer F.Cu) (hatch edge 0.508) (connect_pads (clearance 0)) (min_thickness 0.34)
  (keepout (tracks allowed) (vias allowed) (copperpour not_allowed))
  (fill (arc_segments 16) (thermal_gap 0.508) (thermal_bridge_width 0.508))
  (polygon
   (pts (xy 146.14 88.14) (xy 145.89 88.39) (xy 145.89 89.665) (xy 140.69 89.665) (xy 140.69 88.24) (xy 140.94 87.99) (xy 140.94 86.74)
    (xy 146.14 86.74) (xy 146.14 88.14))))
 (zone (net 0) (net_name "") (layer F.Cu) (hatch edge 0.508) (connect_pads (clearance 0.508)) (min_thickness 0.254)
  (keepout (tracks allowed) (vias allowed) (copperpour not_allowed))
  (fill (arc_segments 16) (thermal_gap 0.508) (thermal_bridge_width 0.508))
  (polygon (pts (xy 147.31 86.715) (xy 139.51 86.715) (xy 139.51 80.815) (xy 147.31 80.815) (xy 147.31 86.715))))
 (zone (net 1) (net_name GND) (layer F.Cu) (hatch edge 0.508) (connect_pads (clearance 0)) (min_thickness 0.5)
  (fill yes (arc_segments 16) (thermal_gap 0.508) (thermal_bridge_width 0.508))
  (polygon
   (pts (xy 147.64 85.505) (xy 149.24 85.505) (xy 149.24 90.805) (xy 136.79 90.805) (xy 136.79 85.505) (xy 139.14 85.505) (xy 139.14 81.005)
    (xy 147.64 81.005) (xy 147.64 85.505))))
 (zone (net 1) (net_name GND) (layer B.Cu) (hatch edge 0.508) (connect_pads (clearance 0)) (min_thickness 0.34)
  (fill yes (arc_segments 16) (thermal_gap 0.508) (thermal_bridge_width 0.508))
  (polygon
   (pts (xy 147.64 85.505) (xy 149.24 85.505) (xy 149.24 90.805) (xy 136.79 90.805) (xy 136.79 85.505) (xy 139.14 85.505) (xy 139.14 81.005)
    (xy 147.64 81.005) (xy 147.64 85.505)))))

